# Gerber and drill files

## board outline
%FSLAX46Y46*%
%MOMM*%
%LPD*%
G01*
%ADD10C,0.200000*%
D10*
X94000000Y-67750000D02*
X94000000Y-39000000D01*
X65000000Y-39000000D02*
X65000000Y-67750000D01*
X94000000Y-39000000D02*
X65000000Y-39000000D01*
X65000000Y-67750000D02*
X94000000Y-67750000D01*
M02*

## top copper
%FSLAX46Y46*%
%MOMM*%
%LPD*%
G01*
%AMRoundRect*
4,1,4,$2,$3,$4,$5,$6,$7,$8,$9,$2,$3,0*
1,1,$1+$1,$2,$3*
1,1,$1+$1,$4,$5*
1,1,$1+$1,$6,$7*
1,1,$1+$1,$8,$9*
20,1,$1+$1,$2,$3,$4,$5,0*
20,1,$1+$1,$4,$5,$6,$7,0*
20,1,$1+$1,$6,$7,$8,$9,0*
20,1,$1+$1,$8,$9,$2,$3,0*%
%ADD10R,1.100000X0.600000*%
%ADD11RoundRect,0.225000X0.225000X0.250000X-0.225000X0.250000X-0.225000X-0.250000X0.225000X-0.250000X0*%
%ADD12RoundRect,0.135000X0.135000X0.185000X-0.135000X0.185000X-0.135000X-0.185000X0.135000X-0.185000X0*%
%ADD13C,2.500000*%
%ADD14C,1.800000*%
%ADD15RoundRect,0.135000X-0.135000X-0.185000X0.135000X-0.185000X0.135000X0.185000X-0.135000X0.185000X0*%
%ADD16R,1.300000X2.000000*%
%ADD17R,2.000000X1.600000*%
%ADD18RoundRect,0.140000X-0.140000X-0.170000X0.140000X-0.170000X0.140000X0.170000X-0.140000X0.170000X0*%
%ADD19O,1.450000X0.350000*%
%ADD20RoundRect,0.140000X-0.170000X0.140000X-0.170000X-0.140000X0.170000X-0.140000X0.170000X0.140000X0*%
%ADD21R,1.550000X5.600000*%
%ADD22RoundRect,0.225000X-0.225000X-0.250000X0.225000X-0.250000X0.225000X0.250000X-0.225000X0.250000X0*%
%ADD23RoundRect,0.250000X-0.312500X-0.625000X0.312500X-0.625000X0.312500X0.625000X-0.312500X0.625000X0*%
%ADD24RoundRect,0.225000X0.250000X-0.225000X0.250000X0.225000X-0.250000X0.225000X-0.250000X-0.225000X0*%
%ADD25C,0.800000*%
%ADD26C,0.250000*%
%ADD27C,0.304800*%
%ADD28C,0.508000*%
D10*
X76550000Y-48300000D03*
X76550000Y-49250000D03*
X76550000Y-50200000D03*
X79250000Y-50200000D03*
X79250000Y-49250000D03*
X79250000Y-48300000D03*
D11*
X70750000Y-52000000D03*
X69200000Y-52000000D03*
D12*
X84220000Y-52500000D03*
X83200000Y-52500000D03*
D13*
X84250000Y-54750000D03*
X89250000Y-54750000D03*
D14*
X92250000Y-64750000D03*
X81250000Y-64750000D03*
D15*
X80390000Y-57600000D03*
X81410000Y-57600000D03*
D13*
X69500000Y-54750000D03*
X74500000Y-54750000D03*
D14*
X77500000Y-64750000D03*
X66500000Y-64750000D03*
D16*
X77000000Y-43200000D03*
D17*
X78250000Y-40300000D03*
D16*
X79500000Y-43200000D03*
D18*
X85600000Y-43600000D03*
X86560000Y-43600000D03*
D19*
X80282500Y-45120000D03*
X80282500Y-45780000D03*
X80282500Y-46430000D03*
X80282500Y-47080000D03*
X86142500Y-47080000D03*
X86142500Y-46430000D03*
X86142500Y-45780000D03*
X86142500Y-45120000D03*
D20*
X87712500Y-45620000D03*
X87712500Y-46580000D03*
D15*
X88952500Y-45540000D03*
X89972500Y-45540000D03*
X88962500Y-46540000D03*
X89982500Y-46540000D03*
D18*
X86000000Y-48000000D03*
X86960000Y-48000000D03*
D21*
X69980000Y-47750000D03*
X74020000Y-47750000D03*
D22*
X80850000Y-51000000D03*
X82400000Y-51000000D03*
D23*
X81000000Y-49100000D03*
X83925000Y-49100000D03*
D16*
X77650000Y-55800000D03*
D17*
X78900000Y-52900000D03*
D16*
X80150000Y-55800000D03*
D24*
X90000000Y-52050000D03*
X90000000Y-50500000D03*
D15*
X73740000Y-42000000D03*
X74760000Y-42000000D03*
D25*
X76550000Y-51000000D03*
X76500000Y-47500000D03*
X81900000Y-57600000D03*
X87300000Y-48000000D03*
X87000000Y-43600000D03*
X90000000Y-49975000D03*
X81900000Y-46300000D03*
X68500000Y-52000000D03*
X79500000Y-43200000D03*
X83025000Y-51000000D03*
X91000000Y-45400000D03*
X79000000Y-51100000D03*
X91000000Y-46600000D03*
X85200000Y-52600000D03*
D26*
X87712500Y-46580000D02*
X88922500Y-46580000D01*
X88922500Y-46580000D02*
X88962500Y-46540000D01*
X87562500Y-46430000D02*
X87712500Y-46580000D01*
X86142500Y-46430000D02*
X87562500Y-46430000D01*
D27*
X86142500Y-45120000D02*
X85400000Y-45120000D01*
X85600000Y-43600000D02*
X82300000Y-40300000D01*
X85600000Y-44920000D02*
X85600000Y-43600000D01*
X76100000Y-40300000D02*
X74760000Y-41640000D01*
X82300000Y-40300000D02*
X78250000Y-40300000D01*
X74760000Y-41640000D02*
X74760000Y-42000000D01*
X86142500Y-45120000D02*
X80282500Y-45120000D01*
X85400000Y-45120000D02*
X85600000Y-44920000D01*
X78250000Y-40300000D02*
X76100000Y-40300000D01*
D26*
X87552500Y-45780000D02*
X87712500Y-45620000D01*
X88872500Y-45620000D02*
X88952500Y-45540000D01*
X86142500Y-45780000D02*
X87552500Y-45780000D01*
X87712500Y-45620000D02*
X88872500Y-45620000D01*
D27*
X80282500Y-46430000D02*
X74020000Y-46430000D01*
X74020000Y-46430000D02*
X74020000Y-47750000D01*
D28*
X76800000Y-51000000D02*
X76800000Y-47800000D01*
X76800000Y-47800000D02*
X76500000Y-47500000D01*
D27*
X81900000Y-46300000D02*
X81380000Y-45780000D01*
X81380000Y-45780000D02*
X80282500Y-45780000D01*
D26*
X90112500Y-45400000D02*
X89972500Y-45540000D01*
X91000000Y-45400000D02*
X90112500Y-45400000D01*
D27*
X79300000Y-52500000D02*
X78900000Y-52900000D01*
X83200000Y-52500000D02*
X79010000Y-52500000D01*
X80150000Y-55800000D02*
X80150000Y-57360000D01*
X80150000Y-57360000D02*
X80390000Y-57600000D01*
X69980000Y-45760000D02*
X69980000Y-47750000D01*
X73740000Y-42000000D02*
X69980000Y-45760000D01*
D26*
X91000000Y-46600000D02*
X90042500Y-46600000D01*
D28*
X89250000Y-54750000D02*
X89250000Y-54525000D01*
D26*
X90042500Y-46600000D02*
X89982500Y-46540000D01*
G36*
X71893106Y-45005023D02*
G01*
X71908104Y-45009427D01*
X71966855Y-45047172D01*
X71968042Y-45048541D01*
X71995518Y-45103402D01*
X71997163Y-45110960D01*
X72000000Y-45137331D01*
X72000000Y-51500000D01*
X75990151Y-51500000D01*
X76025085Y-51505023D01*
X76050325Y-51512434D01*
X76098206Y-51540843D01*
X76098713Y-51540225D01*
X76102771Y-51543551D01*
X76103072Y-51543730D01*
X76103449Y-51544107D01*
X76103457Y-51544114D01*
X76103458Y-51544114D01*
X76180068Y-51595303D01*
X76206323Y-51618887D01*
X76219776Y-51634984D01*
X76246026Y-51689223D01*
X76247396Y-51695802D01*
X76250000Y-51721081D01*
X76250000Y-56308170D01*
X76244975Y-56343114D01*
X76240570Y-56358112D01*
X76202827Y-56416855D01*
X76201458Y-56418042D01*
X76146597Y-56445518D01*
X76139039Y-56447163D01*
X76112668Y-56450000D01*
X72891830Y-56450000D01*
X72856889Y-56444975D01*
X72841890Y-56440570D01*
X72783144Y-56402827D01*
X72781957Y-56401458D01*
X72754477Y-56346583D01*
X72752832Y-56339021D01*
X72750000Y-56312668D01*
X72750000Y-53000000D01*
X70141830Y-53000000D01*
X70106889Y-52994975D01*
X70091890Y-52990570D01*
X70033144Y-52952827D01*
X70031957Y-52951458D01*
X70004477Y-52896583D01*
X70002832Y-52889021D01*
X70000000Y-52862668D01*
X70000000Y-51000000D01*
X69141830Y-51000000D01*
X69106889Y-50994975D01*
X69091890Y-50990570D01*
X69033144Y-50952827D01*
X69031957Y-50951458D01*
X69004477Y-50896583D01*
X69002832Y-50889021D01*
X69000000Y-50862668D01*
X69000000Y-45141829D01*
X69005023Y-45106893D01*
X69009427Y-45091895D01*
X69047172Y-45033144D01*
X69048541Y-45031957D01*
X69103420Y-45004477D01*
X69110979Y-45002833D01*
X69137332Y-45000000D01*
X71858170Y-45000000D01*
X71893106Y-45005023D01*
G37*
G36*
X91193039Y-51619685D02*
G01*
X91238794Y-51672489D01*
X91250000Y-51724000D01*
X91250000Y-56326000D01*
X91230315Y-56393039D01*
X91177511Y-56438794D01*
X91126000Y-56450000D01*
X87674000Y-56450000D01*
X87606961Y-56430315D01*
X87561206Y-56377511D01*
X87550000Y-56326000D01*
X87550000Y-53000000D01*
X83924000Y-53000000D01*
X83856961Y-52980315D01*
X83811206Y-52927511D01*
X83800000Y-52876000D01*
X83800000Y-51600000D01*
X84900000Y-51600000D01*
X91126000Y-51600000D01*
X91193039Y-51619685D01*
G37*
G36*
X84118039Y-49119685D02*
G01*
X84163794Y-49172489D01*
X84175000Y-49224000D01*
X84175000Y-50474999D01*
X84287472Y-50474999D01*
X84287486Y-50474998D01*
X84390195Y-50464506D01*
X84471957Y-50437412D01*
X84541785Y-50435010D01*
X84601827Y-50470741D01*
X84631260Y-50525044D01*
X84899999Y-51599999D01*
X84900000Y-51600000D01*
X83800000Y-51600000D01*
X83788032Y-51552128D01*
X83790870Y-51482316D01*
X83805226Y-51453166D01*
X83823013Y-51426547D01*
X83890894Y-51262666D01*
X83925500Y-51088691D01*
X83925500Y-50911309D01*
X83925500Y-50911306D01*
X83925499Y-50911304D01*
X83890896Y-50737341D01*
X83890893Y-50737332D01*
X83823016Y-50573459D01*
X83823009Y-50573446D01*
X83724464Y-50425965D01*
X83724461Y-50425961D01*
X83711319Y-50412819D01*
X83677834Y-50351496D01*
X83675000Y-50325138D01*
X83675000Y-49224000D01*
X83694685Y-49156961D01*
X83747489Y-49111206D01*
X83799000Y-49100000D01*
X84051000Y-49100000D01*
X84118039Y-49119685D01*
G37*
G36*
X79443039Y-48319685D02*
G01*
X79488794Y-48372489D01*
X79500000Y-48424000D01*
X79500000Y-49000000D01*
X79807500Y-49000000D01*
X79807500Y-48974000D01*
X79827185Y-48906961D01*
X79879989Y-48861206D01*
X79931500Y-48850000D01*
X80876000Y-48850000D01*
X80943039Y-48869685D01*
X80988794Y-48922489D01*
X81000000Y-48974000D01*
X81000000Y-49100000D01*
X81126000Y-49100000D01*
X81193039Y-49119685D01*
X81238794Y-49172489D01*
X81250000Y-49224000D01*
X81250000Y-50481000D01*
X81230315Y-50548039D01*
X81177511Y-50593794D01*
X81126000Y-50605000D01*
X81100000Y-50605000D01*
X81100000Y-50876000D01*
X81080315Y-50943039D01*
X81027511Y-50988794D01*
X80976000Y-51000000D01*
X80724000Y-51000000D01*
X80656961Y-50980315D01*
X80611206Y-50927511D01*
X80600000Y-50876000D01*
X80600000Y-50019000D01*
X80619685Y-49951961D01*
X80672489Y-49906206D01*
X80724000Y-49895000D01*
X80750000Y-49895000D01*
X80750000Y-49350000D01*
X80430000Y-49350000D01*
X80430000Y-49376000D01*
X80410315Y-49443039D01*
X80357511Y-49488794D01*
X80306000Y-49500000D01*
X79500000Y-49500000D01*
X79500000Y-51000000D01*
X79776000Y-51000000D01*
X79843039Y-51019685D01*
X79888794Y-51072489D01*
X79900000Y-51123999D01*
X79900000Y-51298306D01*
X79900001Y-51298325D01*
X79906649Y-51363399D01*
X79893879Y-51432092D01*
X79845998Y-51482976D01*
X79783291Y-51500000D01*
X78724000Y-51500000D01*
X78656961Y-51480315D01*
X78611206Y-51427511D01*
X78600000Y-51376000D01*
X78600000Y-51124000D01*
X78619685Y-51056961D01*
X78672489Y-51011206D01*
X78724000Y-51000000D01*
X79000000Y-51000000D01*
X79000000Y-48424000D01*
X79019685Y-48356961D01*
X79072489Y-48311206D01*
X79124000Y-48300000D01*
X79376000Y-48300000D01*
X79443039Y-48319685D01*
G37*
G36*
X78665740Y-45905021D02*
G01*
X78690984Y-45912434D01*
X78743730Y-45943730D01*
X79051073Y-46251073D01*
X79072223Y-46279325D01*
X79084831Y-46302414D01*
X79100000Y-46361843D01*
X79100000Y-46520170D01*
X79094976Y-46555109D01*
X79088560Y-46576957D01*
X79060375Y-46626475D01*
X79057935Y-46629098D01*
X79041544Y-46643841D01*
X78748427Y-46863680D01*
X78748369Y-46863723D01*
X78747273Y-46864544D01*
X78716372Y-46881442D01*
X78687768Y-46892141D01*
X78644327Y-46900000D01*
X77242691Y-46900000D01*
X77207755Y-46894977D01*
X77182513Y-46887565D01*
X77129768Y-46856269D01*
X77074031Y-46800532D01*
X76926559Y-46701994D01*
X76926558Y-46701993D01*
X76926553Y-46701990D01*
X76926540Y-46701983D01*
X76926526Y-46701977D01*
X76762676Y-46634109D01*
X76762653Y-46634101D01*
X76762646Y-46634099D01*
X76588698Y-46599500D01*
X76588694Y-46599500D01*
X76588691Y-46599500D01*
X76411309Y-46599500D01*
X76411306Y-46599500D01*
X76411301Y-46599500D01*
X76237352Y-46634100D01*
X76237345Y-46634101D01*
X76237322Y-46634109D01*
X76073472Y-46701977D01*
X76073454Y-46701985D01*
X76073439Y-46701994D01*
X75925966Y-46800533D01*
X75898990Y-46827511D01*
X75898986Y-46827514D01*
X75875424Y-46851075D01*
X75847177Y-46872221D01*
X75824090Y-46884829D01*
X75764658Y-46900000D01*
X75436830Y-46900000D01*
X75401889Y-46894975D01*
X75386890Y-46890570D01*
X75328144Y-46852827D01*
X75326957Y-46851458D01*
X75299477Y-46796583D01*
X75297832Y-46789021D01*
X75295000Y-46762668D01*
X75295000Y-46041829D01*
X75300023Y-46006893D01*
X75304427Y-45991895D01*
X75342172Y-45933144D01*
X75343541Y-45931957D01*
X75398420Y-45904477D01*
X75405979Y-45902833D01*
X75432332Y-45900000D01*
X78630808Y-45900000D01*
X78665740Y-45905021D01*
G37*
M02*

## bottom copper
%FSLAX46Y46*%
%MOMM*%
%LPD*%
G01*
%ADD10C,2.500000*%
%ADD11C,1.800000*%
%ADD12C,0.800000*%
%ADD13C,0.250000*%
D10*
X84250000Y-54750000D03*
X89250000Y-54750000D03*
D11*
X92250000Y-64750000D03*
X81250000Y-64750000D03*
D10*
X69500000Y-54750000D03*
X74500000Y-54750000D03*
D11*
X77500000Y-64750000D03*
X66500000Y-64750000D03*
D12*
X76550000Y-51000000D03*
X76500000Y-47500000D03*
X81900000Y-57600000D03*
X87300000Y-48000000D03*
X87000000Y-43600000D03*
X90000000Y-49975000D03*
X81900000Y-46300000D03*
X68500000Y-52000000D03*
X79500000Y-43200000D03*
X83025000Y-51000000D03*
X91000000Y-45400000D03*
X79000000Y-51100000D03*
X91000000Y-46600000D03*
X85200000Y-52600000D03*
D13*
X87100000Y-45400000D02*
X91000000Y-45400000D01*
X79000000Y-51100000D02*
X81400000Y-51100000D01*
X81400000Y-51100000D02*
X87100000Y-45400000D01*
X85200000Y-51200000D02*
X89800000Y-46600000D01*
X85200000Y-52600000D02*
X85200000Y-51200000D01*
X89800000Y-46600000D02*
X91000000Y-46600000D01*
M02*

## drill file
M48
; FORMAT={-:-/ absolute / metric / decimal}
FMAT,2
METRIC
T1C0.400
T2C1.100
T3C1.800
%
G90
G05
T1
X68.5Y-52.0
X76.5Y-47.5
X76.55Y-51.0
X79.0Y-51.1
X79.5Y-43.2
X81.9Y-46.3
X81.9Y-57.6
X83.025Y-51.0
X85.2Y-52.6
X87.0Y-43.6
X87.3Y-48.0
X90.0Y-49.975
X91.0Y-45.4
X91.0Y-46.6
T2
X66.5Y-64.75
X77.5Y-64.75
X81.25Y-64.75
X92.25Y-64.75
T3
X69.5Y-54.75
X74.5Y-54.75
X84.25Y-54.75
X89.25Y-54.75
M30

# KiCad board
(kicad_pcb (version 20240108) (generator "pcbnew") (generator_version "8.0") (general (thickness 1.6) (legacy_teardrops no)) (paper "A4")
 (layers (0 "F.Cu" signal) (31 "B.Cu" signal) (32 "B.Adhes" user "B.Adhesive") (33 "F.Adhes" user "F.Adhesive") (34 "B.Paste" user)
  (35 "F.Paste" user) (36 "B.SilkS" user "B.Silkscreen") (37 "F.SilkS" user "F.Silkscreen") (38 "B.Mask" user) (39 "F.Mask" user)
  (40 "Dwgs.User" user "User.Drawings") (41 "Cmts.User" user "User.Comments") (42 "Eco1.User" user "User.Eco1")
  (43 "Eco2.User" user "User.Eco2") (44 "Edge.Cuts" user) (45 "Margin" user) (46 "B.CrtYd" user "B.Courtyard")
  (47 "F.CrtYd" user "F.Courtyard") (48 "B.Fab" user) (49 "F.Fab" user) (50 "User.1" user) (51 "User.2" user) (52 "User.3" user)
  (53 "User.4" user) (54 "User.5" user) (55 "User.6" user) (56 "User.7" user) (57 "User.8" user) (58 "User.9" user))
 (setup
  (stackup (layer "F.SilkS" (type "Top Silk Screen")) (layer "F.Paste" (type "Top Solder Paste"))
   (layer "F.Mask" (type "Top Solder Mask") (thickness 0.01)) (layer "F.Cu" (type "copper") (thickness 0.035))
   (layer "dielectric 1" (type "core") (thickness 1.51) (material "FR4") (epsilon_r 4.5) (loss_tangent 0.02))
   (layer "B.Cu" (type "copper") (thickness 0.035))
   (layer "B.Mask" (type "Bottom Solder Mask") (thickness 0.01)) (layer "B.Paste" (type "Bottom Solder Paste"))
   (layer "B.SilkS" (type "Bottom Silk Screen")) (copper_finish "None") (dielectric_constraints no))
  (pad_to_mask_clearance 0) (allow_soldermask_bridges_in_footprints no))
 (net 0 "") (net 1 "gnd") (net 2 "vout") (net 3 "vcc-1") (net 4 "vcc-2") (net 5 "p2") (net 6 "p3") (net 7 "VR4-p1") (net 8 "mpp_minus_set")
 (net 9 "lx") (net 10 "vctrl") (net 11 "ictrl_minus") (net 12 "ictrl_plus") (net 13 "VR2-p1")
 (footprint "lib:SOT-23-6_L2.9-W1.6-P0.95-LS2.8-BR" (layer "F.Cu") (at 77.9 49.25 180)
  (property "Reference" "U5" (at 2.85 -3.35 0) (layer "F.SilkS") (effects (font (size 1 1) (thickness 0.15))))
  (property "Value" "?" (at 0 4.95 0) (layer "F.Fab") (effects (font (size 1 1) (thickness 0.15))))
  (pad "1" smd rect (at 1.35 0.95 180) (size 1.1 0.6) (layers "F.Cu" "F.Paste" "F.Mask") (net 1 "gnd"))
  (pad "2" smd rect (at 1.35 0 180) (size 1.1 0.6) (layers "F.Cu" "F.Paste" "F.Mask") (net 1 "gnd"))
  (pad "3" smd rect (at 1.35 -0.95 180) (size 1.1 0.6) (layers "F.Cu" "F.Paste" "F.Mask") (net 1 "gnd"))
  (pad "4" smd rect (at -1.35 -0.95 180) (size 1.1 0.6) (layers "F.Cu" "F.Paste" "F.Mask") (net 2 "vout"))
  (pad "5" smd rect (at -1.35 0 180) (size 1.1 0.6) (layers "F.Cu" "F.Paste" "F.Mask") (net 2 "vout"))
  (pad "6" smd rect (at -1.35 0.95 180) (size 1.1 0.6) (layers "F.Cu" "F.Paste" "F.Mask") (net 2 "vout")))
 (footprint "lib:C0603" (layer "F.Cu") (at 69.975 52 180)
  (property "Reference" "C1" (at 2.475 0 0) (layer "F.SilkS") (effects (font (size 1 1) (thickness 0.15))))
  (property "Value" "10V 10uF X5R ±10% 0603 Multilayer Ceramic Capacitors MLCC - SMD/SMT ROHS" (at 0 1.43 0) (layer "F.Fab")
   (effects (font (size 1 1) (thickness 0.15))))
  (pad "1" smd roundrect (at -0.775 0 180) (size 0.9 0.95) (layers "F.Cu" "F.Paste" "F.Mask") (roundrect_rratio 0.25) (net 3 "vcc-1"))
  (pad "2" smd roundrect (at 0.775 0 180) (size 0.9 0.95) (layers "F.Cu" "F.Paste" "F.Mask") (roundrect_rratio 0.25) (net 1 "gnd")))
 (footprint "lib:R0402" (layer "F.Cu") (at 83.71 52.5 180)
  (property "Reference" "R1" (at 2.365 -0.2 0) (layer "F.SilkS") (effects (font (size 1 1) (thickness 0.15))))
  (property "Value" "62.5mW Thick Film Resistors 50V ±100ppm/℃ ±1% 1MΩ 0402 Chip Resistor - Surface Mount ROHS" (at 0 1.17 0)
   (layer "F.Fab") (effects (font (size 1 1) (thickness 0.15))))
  (pad "1" smd roundrect (at -0.51 0 180) (size 0.54 0.64) (layers "F.Cu" "F.Paste" "F.Mask") (roundrect_rratio 0.25) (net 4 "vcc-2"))
  (pad "2" smd roundrect (at 0.51 0 180) (size 0.54 0.64) (layers "F.Cu" "F.Paste" "F.Mask") (roundrect_rratio 0.25) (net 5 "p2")))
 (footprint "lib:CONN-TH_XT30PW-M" (layer "F.Cu") (at 86.75 59.75)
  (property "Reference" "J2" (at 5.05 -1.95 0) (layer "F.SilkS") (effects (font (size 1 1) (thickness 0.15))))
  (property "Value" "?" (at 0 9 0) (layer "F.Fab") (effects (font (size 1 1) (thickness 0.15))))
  (pad "1" thru_hole circle (at -2.5 -5) (size 2.5 2.5) (drill 1.799996) (layers "*.Cu" "*.Mask") (remove_unused_layers no) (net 1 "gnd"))
  (pad "2" thru_hole circle (at 2.5 -5) (size 2.5 2.5) (drill 1.799996) (layers "*.Cu" "*.Mask") (remove_unused_layers no) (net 4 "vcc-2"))
  (pad "3" thru_hole circle (at 5.5 5) (size 1.8 1.8) (drill 1.100023) (layers "*.Cu" "*.Mask") (remove_unused_layers no))
  (pad "4" thru_hole circle (at -5.5 5) (size 1.8 1.8) (drill 1.100023) (layers "*.Cu" "*.Mask") (remove_unused_layers no)))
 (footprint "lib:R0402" (layer "F.Cu") (at 80.9 57.6)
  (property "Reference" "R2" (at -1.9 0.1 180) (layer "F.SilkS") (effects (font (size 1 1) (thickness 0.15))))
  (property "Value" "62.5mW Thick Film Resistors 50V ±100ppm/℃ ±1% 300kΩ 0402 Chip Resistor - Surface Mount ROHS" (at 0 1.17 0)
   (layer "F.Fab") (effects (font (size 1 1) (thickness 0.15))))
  (pad "1" smd roundrect (at -0.51 0) (size 0.54 0.64) (layers "F.Cu" "F.Paste" "F.Mask") (roundrect_rratio 0.25) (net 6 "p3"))
  (pad "2" smd roundrect (at 0.51 0) (size 0.54 0.64) (layers "F.Cu" "F.Paste" "F.Mask") (roundrect_rratio 0.25) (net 1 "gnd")))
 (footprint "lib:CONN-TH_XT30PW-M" (layer "F.Cu") (at 72 59.75)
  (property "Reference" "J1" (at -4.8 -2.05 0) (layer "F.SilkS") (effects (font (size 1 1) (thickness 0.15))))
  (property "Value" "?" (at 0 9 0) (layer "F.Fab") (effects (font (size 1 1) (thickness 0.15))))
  (pad "1" thru_hole circle (at -2.5 -5) (size 2.5 2.5) (drill 1.799996) (layers "*.Cu" "*.Mask") (remove_unused_layers no) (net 1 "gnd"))
  (pad "2" thru_hole circle (at 2.5 -5) (size 2.5 2.5) (drill 1.799996) (layers "*.Cu" "*.Mask") (remove_unused_layers no) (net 3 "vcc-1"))
  (pad "3" thru_hole circle (at 5.5 5) (size 1.8 1.8) (drill 1.100023) (layers "*.Cu" "*.Mask") (remove_unused_layers no))
  (pad "4" thru_hole circle (at -5.5 5) (size 1.8 1.8) (drill 1.100023) (layers "*.Cu" "*.Mask") (remove_unused_layers no)))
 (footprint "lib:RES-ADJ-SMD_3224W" (layer "F.Cu") (at 78.25 41.75)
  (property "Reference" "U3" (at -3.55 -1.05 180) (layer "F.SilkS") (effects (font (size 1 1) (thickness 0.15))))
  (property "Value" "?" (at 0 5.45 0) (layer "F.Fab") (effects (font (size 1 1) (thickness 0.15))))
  (pad "1" smd rect (at -1.25 1.45 270) (size 2 1.3) (layers "F.Cu" "F.Paste" "F.Mask") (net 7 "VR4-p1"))
  (pad "2" smd rect (at 0 -1.45 270) (size 1.6 2) (layers "F.Cu" "F.Paste" "F.Mask") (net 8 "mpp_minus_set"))
  (pad "3" smd rect (at 1.25 1.45 270) (size 2 1.3) (layers "F.Cu" "F.Paste" "F.Mask") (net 1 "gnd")))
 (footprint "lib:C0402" (layer "F.Cu") (at 86.08 43.6)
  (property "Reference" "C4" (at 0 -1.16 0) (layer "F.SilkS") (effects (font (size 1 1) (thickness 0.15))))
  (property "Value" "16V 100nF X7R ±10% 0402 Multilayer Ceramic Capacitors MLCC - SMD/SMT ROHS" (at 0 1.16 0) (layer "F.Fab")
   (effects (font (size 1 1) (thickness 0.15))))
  (pad "1" smd roundrect (at -0.48 0) (size 0.56 0.62) (layers "F.Cu" "F.Paste" "F.Mask") (roundrect_rratio 0.25) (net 8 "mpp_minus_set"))
  (pad "2" smd roundrect (at 0.48 0) (size 0.56 0.62) (layers "F.Cu" "F.Paste" "F.Mask") (roundrect_rratio 0.25) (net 1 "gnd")))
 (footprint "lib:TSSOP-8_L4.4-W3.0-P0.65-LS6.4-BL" (layer "F.Cu") (at 83.2125 46.1 -90)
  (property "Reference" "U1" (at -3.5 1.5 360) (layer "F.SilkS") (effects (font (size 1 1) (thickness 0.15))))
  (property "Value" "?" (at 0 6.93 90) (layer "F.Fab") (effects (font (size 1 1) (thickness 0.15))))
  (pad "1" smd oval (at -0.98 2.93 270) (size 0.35 1.45) (layers "F.Cu" "F.Paste" "F.Mask") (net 8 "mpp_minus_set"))
  (pad "2" smd oval (at -0.32 2.93 270) (size 0.35 1.45) (layers "F.Cu" "F.Paste" "F.Mask") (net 1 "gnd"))
  (pad "3" smd oval (at 0.33 2.93 270) (size 0.35 1.45) (layers "F.Cu" "F.Paste" "F.Mask") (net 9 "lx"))
  (pad "4" smd oval (at 0.98 2.93 270) (size 0.35 1.45) (layers "F.Cu" "F.Paste" "F.Mask") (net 2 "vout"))
  (pad "5" smd oval (at 0.98 -2.93 270) (size 0.35 1.45) (layers "F.Cu" "F.Paste" "F.Mask") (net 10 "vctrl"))
  (pad "6" smd oval (at 0.33 -2.93 270) (size 0.35 1.45) (layers "F.Cu" "F.Paste" "F.Mask") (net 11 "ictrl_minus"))
  (pad "7" smd oval (at -0.32 -2.93 270) (size 0.35 1.45) (layers "F.Cu" "F.Paste" "F.Mask") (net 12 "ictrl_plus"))
  (pad "8" smd oval (at -0.98 -2.93 270) (size 0.35 1.45) (layers "F.Cu" "F.Paste" "F.Mask") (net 8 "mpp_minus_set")))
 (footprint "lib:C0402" (layer "F.Cu") (at 87.7125 46.1 -90)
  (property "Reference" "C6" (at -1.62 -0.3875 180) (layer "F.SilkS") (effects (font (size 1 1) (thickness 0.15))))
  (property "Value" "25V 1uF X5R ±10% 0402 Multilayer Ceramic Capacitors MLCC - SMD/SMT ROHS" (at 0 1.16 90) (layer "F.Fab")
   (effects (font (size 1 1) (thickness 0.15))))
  (pad "1" smd roundrect (at -0.48 0 270) (size 0.56 0.62) (layers "F.Cu" "F.Paste" "F.Mask") (roundrect_rratio 0.25) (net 12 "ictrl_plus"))
  (pad "2" smd roundrect (at 0.48 0 270) (size 0.56 0.62) (layers "F.Cu" "F.Paste" "F.Mask") (roundrect_rratio 0.25) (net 11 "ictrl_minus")))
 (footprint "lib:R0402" (layer "F.Cu") (at 89.4625 45.54)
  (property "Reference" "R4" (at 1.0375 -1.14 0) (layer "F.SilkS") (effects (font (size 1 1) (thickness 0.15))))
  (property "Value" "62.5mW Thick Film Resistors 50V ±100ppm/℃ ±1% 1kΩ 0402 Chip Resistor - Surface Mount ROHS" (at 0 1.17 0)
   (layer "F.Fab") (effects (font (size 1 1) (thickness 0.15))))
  (pad "1" smd roundrect (at -0.51 0) (size 0.54 0.64) (layers "F.Cu" "F.Paste" "F.Mask") (roundrect_rratio 0.25) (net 12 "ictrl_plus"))
  (pad "2" smd roundrect (at 0.51 0) (size 0.54 0.64) (layers "F.Cu" "F.Paste" "F.Mask") (roundrect_rratio 0.25) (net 2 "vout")))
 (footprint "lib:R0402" (layer "F.Cu") (at 89.4725 46.54)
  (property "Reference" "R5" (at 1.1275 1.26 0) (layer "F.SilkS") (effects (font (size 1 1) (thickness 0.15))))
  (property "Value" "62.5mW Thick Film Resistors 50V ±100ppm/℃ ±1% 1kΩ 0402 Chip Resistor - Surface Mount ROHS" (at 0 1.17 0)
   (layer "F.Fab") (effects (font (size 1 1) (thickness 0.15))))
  (pad "1" smd roundrect (at -0.51 0) (size 0.54 0.64) (layers "F.Cu" "F.Paste" "F.Mask") (roundrect_rratio 0.25) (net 11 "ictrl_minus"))
  (pad "2" smd roundrect (at 0.51 0) (size 0.54 0.64) (layers "F.Cu" "F.Paste" "F.Mask") (roundrect_rratio 0.25) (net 4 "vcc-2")))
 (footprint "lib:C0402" (layer "F.Cu") (at 86.48 48)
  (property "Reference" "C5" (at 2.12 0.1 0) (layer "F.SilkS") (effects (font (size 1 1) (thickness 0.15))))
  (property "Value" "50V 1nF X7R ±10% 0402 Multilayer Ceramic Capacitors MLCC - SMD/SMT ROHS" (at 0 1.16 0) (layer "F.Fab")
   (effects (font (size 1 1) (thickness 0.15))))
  (pad "1" smd roundrect (at -0.48 0) (size 0.56 0.62) (layers "F.Cu" "F.Paste" "F.Mask") (roundrect_rratio 0.25) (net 10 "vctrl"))
  (pad "2" smd roundrect (at 0.48 0) (size 0.56 0.62) (layers "F.Cu" "F.Paste" "F.Mask") (roundrect_rratio 0.25) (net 1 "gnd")))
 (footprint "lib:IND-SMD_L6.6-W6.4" (layer "F.Cu") (at 72 47.75)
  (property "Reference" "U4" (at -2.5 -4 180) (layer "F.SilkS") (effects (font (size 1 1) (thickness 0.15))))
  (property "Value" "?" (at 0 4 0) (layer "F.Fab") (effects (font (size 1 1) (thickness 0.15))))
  (pad "1" smd rect (at -2.02 0) (size 1.55 5.6) (layers "F.Cu" "F.Paste" "F.Mask") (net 3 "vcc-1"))
  (pad "2" smd rect (at 2.02 0) (size 1.55 5.6) (layers "F.Cu" "F.Paste" "F.Mask") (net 9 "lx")))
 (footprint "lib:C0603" (layer "F.Cu") (at 81.625 51)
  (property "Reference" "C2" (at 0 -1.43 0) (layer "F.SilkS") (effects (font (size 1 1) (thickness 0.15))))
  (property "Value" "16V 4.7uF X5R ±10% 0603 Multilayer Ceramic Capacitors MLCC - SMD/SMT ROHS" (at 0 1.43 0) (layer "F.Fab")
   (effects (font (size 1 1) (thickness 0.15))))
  (pad "1" smd roundrect (at -0.775 0) (size 0.9 0.95) (layers "F.Cu" "F.Paste" "F.Mask") (roundrect_rratio 0.25) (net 2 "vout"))
  (pad "2" smd roundrect (at 0.775 0) (size 0.9 0.95) (layers "F.Cu" "F.Paste" "F.Mask") (roundrect_rratio 0.25) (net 1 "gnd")))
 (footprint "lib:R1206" (layer "F.Cu") (at 82.4625 49.1)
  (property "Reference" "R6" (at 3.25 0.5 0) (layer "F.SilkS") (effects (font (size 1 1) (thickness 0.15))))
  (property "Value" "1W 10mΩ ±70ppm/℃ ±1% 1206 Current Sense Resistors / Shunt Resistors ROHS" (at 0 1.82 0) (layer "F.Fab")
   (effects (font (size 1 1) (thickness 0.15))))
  (pad "1" smd roundrect (at -1.4625 0) (size 1.125 1.75) (layers "F.Cu" "F.Paste" "F.Mask") (roundrect_rratio 0.222222) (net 2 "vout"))
  (pad "2" smd roundrect (at 1.4625 0) (size 1.125 1.75) (layers "F.Cu" "F.Paste" "F.Mask") (roundrect_rratio 0.222222) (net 4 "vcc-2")))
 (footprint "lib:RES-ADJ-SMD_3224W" (layer "F.Cu") (at 78.9 54.35)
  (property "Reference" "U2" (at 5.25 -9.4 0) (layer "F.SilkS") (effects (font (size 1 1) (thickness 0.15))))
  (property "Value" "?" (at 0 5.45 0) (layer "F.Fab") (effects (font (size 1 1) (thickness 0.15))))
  (pad "1" smd rect (at -1.25 1.45 270) (size 2 1.3) (layers "F.Cu" "F.Paste" "F.Mask") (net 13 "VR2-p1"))
  (pad "2" smd rect (at 0 -1.45 270) (size 1.6 2) (layers "F.Cu" "F.Paste" "F.Mask") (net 5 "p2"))
  (pad "3" smd rect (at 1.25 1.45 270) (size 2 1.3) (layers "F.Cu" "F.Paste" "F.Mask") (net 6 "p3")))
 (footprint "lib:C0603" (layer "F.Cu") (at 90 51.275 90)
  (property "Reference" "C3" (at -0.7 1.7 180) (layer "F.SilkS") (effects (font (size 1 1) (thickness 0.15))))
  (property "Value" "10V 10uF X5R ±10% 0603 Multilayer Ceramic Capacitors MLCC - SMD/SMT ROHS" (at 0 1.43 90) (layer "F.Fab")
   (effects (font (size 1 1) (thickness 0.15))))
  (pad "1" smd roundrect (at -0.775 0 90) (size 0.9 0.95) (layers "F.Cu" "F.Paste" "F.Mask") (roundrect_rratio 0.25) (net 4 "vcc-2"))
  (pad "2" smd roundrect (at 0.775 0 90) (size 0.9 0.95) (layers "F.Cu" "F.Paste" "F.Mask") (roundrect_rratio 0.25) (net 1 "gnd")))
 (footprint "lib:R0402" (layer "F.Cu") (at 74.25 42)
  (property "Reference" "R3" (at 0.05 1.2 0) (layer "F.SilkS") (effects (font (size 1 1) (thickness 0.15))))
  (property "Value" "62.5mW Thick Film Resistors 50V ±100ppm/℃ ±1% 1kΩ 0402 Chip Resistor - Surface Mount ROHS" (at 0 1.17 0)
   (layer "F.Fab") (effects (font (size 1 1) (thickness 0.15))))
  (pad "1" smd roundrect (at -0.51 0) (size 0.54 0.64) (layers "F.Cu" "F.Paste" "F.Mask") (roundrect_rratio 0.25) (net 3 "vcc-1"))
  (pad "2" smd roundrect (at 0.51 0) (size 0.54 0.64) (layers "F.Cu" "F.Paste" "F.Mask") (roundrect_rratio 0.25) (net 8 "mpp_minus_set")))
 (gr_line (start 94 67.75) (end 94 39) (stroke (width 0.2) (type default)) (layer "Edge.Cuts"))
 (gr_line (start 65 39) (end 65 67.75) (stroke (width 0.2) (type default)) (layer "Edge.Cuts"))
 (gr_line (start 94 39) (end 65 39) (stroke (width 0.2) (type default)) (layer "Edge.Cuts"))
 (gr_line (start 65 67.75) (end 94 67.75) (stroke (width 0.2) (type default)) (layer "Edge.Cuts"))
 (segment (start 87.7125 46.58) (end 88.9225 46.58) (width 0.25) (layer "F.Cu") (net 11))
 (segment (start 88.9225 46.58) (end 88.9625 46.54) (width 0.25) (layer "F.Cu") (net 11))
 (segment (start 87.5625 46.43) (end 87.7125 46.58) (width 0.25) (layer "F.Cu") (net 11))
 (segment (start 86.1425 46.43) (end 87.5625 46.43) (width 0.25) (layer "F.Cu") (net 11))
 (segment (start 86.1425 45.12) (end 85.4 45.12) (width 0.3048) (layer "F.Cu") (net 8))
 (segment (start 85.6 43.6) (end 82.3 40.3) (width 0.3048) (layer "F.Cu") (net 8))
 (segment (start 85.6 44.92) (end 85.6 43.6) (width 0.3048) (layer "F.Cu") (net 8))
 (segment (start 76.1 40.3) (end 74.76 41.64) (width 0.3048) (layer "F.Cu") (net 8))
 (segment (start 82.3 40.3) (end 78.25 40.3) (width 0.3048) (layer "F.Cu") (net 8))
 (segment (start 74.76 41.64) (end 74.76 42) (width 0.3048) (layer "F.Cu") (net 8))
 (segment (start 86.1425 45.12) (end 80.2825 45.12) (width 0.3048) (layer "F.Cu") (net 8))
 (segment (start 85.4 45.12) (end 85.6 44.92) (width 0.3048) (layer "F.Cu") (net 8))
 (segment (start 78.25 40.3) (end 76.1 40.3) (width 0.3048) (layer "F.Cu") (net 8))
 (segment (start 87.5525 45.78) (end 87.7125 45.62) (width 0.25) (layer "F.Cu") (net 12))
 (segment (start 88.8725 45.62) (end 88.9525 45.54) (width 0.25) (layer "F.Cu") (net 12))
 (segment (start 86.1425 45.78) (end 87.5525 45.78) (width 0.25) (layer "F.Cu") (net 12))
 (segment (start 87.7125 45.62) (end 88.8725 45.62) (width 0.25) (layer "F.Cu") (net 12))
 (segment (start 80.2825 46.43) (end 74.02 46.43) (width 0.3048) (layer "F.Cu") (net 9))
 (segment (start 74.02 46.43) (end 74.02 47.75) (width 0.3048) (layer "F.Cu") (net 9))
 (segment (start 76.8 51) (end 76.8 47.8) (width 0.508) (layer "F.Cu") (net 1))
 (segment (start 76.8 47.8) (end 76.5 47.5) (width 0.508) (layer "F.Cu") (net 1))
 (segment (start 81.9 46.3) (end 81.38 45.78) (width 0.3048) (layer "F.Cu") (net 1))
 (segment (start 81.38 45.78) (end 80.2825 45.78) (width 0.3048) (layer "F.Cu") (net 1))
 (via (at 76.55 51) (size 0.8) (drill 0.4) (layers "F.Cu" "B.Cu") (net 1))
 (via (at 76.5 47.5) (size 0.8) (drill 0.4) (layers "F.Cu" "B.Cu") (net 1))
 (via (at 81.9 57.6) (size 0.8) (drill 0.4) (layers "F.Cu" "B.Cu") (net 1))
 (via (at 87.3 48) (size 0.8) (drill 0.4) (layers "F.Cu" "B.Cu") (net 1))
 (via (at 87 43.6) (size 0.8) (drill 0.4) (layers "F.Cu" "B.Cu") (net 1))
 (via (at 90 49.975) (size 0.8) (drill 0.4) (layers "F.Cu" "B.Cu") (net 1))
 (via (at 81.9 46.3) (size 0.8) (drill 0.4) (layers "F.Cu" "B.Cu") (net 1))
 (via (at 68.5 52) (size 0.8) (drill 0.4) (layers "F.Cu" "B.Cu") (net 1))
 (via (at 79.5 43.2) (size 0.8) (drill 0.4) (layers "F.Cu" "B.Cu") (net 1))
 (via (at 83.025 51) (size 0.8) (drill 0.4) (layers "F.Cu" "B.Cu") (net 1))
 (segment (start 90.1125 45.4) (end 89.9725 45.54) (width 0.25) (layer "F.Cu") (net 2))
 (segment (start 91 45.4) (end 90.1125 45.4) (width 0.25) (layer "F.Cu") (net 2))
 (via (at 91 45.4) (size 0.8) (drill 0.4) (layers "F.Cu" "B.Cu") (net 2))
 (via (at 79 51.1) (size 0.8) (drill 0.4) (layers "F.Cu" "B.Cu") (free yes) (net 2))
 (segment (start 87.1 45.4) (end 91 45.4) (width 0.25) (layer "B.Cu") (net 2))
 (segment (start 79 51.1) (end 81.4 51.1) (width 0.25) (layer "B.Cu") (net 2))
 (segment (start 81.4 51.1) (end 87.1 45.4) (width 0.25) (layer "B.Cu") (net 2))
 (segment (start 79.3 52.5) (end 78.9 52.9) (width 0.3048) (layer "F.Cu") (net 5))
 (segment (start 83.2 52.5) (end 79.01 52.5) (width 0.3048) (layer "F.Cu") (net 5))
 (segment (start 80.15 55.8) (end 80.15 57.36) (width 0.3048) (layer "F.Cu") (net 6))
 (segment (start 80.15 57.36) (end 80.39 57.6) (width 0.3048) (layer "F.Cu") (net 6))
 (segment (start 69.98 45.76) (end 69.98 47.75) (width 0.3048) (layer "F.Cu") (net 3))
 (segment (start 73.74 42) (end 69.98 45.76) (width 0.3048) (layer "F.Cu") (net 3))
 (segment (start 91 46.6) (end 90.0425 46.6) (width 0.25) (layer "F.Cu") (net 4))
 (segment (start 89.25 54.75) (end 89.25 54.525) (width 0.508) (layer "F.Cu") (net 4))
 (segment (start 90.0425 46.6) (end 89.9825 46.54) (width 0.25) (layer "F.Cu") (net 4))
 (via (at 91 46.6) (size 0.8) (drill 0.4) (layers "F.Cu" "B.Cu") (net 4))
 (via (at 85.2 52.6) (size 0.8) (drill 0.4) (layers "F.Cu" "B.Cu") (free yes) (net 4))
 (segment (start 85.2 51.2) (end 89.8 46.6) (width 0.25) (layer "B.Cu") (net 4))
 (segment (start 85.2 52.6) (end 85.2 51.2) (width 0.25) (layer "B.Cu") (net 4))
 (segment (start 89.8 46.6) (end 91 46.6) (width 0.25) (layer "B.Cu") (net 4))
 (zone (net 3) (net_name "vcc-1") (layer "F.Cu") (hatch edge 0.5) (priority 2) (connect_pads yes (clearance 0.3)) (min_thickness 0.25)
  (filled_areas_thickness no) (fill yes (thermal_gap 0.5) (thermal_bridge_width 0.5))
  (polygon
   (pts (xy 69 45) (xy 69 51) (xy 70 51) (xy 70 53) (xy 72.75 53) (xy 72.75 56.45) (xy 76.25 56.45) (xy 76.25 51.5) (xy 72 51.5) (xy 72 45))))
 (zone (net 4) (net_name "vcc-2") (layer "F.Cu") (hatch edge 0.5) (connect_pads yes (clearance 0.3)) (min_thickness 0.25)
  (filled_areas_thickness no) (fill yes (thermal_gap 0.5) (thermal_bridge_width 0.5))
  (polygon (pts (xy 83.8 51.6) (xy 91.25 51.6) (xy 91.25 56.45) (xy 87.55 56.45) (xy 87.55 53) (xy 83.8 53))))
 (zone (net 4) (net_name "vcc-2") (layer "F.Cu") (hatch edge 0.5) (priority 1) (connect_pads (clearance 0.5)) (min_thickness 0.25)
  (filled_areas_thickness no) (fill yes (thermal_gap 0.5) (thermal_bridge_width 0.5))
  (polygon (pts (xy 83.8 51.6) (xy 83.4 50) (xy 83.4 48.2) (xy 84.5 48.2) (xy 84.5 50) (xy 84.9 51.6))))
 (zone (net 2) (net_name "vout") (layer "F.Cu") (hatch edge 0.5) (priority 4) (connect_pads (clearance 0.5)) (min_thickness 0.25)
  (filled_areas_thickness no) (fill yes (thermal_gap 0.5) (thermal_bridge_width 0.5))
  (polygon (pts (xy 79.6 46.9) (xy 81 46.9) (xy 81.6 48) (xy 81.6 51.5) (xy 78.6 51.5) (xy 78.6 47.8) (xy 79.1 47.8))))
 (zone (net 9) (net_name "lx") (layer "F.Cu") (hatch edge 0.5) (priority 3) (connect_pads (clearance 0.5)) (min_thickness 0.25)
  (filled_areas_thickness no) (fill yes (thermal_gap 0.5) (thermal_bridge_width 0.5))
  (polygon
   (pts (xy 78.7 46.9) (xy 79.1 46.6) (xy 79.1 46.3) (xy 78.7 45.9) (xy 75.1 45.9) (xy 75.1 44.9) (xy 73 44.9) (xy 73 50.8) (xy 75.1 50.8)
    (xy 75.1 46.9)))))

